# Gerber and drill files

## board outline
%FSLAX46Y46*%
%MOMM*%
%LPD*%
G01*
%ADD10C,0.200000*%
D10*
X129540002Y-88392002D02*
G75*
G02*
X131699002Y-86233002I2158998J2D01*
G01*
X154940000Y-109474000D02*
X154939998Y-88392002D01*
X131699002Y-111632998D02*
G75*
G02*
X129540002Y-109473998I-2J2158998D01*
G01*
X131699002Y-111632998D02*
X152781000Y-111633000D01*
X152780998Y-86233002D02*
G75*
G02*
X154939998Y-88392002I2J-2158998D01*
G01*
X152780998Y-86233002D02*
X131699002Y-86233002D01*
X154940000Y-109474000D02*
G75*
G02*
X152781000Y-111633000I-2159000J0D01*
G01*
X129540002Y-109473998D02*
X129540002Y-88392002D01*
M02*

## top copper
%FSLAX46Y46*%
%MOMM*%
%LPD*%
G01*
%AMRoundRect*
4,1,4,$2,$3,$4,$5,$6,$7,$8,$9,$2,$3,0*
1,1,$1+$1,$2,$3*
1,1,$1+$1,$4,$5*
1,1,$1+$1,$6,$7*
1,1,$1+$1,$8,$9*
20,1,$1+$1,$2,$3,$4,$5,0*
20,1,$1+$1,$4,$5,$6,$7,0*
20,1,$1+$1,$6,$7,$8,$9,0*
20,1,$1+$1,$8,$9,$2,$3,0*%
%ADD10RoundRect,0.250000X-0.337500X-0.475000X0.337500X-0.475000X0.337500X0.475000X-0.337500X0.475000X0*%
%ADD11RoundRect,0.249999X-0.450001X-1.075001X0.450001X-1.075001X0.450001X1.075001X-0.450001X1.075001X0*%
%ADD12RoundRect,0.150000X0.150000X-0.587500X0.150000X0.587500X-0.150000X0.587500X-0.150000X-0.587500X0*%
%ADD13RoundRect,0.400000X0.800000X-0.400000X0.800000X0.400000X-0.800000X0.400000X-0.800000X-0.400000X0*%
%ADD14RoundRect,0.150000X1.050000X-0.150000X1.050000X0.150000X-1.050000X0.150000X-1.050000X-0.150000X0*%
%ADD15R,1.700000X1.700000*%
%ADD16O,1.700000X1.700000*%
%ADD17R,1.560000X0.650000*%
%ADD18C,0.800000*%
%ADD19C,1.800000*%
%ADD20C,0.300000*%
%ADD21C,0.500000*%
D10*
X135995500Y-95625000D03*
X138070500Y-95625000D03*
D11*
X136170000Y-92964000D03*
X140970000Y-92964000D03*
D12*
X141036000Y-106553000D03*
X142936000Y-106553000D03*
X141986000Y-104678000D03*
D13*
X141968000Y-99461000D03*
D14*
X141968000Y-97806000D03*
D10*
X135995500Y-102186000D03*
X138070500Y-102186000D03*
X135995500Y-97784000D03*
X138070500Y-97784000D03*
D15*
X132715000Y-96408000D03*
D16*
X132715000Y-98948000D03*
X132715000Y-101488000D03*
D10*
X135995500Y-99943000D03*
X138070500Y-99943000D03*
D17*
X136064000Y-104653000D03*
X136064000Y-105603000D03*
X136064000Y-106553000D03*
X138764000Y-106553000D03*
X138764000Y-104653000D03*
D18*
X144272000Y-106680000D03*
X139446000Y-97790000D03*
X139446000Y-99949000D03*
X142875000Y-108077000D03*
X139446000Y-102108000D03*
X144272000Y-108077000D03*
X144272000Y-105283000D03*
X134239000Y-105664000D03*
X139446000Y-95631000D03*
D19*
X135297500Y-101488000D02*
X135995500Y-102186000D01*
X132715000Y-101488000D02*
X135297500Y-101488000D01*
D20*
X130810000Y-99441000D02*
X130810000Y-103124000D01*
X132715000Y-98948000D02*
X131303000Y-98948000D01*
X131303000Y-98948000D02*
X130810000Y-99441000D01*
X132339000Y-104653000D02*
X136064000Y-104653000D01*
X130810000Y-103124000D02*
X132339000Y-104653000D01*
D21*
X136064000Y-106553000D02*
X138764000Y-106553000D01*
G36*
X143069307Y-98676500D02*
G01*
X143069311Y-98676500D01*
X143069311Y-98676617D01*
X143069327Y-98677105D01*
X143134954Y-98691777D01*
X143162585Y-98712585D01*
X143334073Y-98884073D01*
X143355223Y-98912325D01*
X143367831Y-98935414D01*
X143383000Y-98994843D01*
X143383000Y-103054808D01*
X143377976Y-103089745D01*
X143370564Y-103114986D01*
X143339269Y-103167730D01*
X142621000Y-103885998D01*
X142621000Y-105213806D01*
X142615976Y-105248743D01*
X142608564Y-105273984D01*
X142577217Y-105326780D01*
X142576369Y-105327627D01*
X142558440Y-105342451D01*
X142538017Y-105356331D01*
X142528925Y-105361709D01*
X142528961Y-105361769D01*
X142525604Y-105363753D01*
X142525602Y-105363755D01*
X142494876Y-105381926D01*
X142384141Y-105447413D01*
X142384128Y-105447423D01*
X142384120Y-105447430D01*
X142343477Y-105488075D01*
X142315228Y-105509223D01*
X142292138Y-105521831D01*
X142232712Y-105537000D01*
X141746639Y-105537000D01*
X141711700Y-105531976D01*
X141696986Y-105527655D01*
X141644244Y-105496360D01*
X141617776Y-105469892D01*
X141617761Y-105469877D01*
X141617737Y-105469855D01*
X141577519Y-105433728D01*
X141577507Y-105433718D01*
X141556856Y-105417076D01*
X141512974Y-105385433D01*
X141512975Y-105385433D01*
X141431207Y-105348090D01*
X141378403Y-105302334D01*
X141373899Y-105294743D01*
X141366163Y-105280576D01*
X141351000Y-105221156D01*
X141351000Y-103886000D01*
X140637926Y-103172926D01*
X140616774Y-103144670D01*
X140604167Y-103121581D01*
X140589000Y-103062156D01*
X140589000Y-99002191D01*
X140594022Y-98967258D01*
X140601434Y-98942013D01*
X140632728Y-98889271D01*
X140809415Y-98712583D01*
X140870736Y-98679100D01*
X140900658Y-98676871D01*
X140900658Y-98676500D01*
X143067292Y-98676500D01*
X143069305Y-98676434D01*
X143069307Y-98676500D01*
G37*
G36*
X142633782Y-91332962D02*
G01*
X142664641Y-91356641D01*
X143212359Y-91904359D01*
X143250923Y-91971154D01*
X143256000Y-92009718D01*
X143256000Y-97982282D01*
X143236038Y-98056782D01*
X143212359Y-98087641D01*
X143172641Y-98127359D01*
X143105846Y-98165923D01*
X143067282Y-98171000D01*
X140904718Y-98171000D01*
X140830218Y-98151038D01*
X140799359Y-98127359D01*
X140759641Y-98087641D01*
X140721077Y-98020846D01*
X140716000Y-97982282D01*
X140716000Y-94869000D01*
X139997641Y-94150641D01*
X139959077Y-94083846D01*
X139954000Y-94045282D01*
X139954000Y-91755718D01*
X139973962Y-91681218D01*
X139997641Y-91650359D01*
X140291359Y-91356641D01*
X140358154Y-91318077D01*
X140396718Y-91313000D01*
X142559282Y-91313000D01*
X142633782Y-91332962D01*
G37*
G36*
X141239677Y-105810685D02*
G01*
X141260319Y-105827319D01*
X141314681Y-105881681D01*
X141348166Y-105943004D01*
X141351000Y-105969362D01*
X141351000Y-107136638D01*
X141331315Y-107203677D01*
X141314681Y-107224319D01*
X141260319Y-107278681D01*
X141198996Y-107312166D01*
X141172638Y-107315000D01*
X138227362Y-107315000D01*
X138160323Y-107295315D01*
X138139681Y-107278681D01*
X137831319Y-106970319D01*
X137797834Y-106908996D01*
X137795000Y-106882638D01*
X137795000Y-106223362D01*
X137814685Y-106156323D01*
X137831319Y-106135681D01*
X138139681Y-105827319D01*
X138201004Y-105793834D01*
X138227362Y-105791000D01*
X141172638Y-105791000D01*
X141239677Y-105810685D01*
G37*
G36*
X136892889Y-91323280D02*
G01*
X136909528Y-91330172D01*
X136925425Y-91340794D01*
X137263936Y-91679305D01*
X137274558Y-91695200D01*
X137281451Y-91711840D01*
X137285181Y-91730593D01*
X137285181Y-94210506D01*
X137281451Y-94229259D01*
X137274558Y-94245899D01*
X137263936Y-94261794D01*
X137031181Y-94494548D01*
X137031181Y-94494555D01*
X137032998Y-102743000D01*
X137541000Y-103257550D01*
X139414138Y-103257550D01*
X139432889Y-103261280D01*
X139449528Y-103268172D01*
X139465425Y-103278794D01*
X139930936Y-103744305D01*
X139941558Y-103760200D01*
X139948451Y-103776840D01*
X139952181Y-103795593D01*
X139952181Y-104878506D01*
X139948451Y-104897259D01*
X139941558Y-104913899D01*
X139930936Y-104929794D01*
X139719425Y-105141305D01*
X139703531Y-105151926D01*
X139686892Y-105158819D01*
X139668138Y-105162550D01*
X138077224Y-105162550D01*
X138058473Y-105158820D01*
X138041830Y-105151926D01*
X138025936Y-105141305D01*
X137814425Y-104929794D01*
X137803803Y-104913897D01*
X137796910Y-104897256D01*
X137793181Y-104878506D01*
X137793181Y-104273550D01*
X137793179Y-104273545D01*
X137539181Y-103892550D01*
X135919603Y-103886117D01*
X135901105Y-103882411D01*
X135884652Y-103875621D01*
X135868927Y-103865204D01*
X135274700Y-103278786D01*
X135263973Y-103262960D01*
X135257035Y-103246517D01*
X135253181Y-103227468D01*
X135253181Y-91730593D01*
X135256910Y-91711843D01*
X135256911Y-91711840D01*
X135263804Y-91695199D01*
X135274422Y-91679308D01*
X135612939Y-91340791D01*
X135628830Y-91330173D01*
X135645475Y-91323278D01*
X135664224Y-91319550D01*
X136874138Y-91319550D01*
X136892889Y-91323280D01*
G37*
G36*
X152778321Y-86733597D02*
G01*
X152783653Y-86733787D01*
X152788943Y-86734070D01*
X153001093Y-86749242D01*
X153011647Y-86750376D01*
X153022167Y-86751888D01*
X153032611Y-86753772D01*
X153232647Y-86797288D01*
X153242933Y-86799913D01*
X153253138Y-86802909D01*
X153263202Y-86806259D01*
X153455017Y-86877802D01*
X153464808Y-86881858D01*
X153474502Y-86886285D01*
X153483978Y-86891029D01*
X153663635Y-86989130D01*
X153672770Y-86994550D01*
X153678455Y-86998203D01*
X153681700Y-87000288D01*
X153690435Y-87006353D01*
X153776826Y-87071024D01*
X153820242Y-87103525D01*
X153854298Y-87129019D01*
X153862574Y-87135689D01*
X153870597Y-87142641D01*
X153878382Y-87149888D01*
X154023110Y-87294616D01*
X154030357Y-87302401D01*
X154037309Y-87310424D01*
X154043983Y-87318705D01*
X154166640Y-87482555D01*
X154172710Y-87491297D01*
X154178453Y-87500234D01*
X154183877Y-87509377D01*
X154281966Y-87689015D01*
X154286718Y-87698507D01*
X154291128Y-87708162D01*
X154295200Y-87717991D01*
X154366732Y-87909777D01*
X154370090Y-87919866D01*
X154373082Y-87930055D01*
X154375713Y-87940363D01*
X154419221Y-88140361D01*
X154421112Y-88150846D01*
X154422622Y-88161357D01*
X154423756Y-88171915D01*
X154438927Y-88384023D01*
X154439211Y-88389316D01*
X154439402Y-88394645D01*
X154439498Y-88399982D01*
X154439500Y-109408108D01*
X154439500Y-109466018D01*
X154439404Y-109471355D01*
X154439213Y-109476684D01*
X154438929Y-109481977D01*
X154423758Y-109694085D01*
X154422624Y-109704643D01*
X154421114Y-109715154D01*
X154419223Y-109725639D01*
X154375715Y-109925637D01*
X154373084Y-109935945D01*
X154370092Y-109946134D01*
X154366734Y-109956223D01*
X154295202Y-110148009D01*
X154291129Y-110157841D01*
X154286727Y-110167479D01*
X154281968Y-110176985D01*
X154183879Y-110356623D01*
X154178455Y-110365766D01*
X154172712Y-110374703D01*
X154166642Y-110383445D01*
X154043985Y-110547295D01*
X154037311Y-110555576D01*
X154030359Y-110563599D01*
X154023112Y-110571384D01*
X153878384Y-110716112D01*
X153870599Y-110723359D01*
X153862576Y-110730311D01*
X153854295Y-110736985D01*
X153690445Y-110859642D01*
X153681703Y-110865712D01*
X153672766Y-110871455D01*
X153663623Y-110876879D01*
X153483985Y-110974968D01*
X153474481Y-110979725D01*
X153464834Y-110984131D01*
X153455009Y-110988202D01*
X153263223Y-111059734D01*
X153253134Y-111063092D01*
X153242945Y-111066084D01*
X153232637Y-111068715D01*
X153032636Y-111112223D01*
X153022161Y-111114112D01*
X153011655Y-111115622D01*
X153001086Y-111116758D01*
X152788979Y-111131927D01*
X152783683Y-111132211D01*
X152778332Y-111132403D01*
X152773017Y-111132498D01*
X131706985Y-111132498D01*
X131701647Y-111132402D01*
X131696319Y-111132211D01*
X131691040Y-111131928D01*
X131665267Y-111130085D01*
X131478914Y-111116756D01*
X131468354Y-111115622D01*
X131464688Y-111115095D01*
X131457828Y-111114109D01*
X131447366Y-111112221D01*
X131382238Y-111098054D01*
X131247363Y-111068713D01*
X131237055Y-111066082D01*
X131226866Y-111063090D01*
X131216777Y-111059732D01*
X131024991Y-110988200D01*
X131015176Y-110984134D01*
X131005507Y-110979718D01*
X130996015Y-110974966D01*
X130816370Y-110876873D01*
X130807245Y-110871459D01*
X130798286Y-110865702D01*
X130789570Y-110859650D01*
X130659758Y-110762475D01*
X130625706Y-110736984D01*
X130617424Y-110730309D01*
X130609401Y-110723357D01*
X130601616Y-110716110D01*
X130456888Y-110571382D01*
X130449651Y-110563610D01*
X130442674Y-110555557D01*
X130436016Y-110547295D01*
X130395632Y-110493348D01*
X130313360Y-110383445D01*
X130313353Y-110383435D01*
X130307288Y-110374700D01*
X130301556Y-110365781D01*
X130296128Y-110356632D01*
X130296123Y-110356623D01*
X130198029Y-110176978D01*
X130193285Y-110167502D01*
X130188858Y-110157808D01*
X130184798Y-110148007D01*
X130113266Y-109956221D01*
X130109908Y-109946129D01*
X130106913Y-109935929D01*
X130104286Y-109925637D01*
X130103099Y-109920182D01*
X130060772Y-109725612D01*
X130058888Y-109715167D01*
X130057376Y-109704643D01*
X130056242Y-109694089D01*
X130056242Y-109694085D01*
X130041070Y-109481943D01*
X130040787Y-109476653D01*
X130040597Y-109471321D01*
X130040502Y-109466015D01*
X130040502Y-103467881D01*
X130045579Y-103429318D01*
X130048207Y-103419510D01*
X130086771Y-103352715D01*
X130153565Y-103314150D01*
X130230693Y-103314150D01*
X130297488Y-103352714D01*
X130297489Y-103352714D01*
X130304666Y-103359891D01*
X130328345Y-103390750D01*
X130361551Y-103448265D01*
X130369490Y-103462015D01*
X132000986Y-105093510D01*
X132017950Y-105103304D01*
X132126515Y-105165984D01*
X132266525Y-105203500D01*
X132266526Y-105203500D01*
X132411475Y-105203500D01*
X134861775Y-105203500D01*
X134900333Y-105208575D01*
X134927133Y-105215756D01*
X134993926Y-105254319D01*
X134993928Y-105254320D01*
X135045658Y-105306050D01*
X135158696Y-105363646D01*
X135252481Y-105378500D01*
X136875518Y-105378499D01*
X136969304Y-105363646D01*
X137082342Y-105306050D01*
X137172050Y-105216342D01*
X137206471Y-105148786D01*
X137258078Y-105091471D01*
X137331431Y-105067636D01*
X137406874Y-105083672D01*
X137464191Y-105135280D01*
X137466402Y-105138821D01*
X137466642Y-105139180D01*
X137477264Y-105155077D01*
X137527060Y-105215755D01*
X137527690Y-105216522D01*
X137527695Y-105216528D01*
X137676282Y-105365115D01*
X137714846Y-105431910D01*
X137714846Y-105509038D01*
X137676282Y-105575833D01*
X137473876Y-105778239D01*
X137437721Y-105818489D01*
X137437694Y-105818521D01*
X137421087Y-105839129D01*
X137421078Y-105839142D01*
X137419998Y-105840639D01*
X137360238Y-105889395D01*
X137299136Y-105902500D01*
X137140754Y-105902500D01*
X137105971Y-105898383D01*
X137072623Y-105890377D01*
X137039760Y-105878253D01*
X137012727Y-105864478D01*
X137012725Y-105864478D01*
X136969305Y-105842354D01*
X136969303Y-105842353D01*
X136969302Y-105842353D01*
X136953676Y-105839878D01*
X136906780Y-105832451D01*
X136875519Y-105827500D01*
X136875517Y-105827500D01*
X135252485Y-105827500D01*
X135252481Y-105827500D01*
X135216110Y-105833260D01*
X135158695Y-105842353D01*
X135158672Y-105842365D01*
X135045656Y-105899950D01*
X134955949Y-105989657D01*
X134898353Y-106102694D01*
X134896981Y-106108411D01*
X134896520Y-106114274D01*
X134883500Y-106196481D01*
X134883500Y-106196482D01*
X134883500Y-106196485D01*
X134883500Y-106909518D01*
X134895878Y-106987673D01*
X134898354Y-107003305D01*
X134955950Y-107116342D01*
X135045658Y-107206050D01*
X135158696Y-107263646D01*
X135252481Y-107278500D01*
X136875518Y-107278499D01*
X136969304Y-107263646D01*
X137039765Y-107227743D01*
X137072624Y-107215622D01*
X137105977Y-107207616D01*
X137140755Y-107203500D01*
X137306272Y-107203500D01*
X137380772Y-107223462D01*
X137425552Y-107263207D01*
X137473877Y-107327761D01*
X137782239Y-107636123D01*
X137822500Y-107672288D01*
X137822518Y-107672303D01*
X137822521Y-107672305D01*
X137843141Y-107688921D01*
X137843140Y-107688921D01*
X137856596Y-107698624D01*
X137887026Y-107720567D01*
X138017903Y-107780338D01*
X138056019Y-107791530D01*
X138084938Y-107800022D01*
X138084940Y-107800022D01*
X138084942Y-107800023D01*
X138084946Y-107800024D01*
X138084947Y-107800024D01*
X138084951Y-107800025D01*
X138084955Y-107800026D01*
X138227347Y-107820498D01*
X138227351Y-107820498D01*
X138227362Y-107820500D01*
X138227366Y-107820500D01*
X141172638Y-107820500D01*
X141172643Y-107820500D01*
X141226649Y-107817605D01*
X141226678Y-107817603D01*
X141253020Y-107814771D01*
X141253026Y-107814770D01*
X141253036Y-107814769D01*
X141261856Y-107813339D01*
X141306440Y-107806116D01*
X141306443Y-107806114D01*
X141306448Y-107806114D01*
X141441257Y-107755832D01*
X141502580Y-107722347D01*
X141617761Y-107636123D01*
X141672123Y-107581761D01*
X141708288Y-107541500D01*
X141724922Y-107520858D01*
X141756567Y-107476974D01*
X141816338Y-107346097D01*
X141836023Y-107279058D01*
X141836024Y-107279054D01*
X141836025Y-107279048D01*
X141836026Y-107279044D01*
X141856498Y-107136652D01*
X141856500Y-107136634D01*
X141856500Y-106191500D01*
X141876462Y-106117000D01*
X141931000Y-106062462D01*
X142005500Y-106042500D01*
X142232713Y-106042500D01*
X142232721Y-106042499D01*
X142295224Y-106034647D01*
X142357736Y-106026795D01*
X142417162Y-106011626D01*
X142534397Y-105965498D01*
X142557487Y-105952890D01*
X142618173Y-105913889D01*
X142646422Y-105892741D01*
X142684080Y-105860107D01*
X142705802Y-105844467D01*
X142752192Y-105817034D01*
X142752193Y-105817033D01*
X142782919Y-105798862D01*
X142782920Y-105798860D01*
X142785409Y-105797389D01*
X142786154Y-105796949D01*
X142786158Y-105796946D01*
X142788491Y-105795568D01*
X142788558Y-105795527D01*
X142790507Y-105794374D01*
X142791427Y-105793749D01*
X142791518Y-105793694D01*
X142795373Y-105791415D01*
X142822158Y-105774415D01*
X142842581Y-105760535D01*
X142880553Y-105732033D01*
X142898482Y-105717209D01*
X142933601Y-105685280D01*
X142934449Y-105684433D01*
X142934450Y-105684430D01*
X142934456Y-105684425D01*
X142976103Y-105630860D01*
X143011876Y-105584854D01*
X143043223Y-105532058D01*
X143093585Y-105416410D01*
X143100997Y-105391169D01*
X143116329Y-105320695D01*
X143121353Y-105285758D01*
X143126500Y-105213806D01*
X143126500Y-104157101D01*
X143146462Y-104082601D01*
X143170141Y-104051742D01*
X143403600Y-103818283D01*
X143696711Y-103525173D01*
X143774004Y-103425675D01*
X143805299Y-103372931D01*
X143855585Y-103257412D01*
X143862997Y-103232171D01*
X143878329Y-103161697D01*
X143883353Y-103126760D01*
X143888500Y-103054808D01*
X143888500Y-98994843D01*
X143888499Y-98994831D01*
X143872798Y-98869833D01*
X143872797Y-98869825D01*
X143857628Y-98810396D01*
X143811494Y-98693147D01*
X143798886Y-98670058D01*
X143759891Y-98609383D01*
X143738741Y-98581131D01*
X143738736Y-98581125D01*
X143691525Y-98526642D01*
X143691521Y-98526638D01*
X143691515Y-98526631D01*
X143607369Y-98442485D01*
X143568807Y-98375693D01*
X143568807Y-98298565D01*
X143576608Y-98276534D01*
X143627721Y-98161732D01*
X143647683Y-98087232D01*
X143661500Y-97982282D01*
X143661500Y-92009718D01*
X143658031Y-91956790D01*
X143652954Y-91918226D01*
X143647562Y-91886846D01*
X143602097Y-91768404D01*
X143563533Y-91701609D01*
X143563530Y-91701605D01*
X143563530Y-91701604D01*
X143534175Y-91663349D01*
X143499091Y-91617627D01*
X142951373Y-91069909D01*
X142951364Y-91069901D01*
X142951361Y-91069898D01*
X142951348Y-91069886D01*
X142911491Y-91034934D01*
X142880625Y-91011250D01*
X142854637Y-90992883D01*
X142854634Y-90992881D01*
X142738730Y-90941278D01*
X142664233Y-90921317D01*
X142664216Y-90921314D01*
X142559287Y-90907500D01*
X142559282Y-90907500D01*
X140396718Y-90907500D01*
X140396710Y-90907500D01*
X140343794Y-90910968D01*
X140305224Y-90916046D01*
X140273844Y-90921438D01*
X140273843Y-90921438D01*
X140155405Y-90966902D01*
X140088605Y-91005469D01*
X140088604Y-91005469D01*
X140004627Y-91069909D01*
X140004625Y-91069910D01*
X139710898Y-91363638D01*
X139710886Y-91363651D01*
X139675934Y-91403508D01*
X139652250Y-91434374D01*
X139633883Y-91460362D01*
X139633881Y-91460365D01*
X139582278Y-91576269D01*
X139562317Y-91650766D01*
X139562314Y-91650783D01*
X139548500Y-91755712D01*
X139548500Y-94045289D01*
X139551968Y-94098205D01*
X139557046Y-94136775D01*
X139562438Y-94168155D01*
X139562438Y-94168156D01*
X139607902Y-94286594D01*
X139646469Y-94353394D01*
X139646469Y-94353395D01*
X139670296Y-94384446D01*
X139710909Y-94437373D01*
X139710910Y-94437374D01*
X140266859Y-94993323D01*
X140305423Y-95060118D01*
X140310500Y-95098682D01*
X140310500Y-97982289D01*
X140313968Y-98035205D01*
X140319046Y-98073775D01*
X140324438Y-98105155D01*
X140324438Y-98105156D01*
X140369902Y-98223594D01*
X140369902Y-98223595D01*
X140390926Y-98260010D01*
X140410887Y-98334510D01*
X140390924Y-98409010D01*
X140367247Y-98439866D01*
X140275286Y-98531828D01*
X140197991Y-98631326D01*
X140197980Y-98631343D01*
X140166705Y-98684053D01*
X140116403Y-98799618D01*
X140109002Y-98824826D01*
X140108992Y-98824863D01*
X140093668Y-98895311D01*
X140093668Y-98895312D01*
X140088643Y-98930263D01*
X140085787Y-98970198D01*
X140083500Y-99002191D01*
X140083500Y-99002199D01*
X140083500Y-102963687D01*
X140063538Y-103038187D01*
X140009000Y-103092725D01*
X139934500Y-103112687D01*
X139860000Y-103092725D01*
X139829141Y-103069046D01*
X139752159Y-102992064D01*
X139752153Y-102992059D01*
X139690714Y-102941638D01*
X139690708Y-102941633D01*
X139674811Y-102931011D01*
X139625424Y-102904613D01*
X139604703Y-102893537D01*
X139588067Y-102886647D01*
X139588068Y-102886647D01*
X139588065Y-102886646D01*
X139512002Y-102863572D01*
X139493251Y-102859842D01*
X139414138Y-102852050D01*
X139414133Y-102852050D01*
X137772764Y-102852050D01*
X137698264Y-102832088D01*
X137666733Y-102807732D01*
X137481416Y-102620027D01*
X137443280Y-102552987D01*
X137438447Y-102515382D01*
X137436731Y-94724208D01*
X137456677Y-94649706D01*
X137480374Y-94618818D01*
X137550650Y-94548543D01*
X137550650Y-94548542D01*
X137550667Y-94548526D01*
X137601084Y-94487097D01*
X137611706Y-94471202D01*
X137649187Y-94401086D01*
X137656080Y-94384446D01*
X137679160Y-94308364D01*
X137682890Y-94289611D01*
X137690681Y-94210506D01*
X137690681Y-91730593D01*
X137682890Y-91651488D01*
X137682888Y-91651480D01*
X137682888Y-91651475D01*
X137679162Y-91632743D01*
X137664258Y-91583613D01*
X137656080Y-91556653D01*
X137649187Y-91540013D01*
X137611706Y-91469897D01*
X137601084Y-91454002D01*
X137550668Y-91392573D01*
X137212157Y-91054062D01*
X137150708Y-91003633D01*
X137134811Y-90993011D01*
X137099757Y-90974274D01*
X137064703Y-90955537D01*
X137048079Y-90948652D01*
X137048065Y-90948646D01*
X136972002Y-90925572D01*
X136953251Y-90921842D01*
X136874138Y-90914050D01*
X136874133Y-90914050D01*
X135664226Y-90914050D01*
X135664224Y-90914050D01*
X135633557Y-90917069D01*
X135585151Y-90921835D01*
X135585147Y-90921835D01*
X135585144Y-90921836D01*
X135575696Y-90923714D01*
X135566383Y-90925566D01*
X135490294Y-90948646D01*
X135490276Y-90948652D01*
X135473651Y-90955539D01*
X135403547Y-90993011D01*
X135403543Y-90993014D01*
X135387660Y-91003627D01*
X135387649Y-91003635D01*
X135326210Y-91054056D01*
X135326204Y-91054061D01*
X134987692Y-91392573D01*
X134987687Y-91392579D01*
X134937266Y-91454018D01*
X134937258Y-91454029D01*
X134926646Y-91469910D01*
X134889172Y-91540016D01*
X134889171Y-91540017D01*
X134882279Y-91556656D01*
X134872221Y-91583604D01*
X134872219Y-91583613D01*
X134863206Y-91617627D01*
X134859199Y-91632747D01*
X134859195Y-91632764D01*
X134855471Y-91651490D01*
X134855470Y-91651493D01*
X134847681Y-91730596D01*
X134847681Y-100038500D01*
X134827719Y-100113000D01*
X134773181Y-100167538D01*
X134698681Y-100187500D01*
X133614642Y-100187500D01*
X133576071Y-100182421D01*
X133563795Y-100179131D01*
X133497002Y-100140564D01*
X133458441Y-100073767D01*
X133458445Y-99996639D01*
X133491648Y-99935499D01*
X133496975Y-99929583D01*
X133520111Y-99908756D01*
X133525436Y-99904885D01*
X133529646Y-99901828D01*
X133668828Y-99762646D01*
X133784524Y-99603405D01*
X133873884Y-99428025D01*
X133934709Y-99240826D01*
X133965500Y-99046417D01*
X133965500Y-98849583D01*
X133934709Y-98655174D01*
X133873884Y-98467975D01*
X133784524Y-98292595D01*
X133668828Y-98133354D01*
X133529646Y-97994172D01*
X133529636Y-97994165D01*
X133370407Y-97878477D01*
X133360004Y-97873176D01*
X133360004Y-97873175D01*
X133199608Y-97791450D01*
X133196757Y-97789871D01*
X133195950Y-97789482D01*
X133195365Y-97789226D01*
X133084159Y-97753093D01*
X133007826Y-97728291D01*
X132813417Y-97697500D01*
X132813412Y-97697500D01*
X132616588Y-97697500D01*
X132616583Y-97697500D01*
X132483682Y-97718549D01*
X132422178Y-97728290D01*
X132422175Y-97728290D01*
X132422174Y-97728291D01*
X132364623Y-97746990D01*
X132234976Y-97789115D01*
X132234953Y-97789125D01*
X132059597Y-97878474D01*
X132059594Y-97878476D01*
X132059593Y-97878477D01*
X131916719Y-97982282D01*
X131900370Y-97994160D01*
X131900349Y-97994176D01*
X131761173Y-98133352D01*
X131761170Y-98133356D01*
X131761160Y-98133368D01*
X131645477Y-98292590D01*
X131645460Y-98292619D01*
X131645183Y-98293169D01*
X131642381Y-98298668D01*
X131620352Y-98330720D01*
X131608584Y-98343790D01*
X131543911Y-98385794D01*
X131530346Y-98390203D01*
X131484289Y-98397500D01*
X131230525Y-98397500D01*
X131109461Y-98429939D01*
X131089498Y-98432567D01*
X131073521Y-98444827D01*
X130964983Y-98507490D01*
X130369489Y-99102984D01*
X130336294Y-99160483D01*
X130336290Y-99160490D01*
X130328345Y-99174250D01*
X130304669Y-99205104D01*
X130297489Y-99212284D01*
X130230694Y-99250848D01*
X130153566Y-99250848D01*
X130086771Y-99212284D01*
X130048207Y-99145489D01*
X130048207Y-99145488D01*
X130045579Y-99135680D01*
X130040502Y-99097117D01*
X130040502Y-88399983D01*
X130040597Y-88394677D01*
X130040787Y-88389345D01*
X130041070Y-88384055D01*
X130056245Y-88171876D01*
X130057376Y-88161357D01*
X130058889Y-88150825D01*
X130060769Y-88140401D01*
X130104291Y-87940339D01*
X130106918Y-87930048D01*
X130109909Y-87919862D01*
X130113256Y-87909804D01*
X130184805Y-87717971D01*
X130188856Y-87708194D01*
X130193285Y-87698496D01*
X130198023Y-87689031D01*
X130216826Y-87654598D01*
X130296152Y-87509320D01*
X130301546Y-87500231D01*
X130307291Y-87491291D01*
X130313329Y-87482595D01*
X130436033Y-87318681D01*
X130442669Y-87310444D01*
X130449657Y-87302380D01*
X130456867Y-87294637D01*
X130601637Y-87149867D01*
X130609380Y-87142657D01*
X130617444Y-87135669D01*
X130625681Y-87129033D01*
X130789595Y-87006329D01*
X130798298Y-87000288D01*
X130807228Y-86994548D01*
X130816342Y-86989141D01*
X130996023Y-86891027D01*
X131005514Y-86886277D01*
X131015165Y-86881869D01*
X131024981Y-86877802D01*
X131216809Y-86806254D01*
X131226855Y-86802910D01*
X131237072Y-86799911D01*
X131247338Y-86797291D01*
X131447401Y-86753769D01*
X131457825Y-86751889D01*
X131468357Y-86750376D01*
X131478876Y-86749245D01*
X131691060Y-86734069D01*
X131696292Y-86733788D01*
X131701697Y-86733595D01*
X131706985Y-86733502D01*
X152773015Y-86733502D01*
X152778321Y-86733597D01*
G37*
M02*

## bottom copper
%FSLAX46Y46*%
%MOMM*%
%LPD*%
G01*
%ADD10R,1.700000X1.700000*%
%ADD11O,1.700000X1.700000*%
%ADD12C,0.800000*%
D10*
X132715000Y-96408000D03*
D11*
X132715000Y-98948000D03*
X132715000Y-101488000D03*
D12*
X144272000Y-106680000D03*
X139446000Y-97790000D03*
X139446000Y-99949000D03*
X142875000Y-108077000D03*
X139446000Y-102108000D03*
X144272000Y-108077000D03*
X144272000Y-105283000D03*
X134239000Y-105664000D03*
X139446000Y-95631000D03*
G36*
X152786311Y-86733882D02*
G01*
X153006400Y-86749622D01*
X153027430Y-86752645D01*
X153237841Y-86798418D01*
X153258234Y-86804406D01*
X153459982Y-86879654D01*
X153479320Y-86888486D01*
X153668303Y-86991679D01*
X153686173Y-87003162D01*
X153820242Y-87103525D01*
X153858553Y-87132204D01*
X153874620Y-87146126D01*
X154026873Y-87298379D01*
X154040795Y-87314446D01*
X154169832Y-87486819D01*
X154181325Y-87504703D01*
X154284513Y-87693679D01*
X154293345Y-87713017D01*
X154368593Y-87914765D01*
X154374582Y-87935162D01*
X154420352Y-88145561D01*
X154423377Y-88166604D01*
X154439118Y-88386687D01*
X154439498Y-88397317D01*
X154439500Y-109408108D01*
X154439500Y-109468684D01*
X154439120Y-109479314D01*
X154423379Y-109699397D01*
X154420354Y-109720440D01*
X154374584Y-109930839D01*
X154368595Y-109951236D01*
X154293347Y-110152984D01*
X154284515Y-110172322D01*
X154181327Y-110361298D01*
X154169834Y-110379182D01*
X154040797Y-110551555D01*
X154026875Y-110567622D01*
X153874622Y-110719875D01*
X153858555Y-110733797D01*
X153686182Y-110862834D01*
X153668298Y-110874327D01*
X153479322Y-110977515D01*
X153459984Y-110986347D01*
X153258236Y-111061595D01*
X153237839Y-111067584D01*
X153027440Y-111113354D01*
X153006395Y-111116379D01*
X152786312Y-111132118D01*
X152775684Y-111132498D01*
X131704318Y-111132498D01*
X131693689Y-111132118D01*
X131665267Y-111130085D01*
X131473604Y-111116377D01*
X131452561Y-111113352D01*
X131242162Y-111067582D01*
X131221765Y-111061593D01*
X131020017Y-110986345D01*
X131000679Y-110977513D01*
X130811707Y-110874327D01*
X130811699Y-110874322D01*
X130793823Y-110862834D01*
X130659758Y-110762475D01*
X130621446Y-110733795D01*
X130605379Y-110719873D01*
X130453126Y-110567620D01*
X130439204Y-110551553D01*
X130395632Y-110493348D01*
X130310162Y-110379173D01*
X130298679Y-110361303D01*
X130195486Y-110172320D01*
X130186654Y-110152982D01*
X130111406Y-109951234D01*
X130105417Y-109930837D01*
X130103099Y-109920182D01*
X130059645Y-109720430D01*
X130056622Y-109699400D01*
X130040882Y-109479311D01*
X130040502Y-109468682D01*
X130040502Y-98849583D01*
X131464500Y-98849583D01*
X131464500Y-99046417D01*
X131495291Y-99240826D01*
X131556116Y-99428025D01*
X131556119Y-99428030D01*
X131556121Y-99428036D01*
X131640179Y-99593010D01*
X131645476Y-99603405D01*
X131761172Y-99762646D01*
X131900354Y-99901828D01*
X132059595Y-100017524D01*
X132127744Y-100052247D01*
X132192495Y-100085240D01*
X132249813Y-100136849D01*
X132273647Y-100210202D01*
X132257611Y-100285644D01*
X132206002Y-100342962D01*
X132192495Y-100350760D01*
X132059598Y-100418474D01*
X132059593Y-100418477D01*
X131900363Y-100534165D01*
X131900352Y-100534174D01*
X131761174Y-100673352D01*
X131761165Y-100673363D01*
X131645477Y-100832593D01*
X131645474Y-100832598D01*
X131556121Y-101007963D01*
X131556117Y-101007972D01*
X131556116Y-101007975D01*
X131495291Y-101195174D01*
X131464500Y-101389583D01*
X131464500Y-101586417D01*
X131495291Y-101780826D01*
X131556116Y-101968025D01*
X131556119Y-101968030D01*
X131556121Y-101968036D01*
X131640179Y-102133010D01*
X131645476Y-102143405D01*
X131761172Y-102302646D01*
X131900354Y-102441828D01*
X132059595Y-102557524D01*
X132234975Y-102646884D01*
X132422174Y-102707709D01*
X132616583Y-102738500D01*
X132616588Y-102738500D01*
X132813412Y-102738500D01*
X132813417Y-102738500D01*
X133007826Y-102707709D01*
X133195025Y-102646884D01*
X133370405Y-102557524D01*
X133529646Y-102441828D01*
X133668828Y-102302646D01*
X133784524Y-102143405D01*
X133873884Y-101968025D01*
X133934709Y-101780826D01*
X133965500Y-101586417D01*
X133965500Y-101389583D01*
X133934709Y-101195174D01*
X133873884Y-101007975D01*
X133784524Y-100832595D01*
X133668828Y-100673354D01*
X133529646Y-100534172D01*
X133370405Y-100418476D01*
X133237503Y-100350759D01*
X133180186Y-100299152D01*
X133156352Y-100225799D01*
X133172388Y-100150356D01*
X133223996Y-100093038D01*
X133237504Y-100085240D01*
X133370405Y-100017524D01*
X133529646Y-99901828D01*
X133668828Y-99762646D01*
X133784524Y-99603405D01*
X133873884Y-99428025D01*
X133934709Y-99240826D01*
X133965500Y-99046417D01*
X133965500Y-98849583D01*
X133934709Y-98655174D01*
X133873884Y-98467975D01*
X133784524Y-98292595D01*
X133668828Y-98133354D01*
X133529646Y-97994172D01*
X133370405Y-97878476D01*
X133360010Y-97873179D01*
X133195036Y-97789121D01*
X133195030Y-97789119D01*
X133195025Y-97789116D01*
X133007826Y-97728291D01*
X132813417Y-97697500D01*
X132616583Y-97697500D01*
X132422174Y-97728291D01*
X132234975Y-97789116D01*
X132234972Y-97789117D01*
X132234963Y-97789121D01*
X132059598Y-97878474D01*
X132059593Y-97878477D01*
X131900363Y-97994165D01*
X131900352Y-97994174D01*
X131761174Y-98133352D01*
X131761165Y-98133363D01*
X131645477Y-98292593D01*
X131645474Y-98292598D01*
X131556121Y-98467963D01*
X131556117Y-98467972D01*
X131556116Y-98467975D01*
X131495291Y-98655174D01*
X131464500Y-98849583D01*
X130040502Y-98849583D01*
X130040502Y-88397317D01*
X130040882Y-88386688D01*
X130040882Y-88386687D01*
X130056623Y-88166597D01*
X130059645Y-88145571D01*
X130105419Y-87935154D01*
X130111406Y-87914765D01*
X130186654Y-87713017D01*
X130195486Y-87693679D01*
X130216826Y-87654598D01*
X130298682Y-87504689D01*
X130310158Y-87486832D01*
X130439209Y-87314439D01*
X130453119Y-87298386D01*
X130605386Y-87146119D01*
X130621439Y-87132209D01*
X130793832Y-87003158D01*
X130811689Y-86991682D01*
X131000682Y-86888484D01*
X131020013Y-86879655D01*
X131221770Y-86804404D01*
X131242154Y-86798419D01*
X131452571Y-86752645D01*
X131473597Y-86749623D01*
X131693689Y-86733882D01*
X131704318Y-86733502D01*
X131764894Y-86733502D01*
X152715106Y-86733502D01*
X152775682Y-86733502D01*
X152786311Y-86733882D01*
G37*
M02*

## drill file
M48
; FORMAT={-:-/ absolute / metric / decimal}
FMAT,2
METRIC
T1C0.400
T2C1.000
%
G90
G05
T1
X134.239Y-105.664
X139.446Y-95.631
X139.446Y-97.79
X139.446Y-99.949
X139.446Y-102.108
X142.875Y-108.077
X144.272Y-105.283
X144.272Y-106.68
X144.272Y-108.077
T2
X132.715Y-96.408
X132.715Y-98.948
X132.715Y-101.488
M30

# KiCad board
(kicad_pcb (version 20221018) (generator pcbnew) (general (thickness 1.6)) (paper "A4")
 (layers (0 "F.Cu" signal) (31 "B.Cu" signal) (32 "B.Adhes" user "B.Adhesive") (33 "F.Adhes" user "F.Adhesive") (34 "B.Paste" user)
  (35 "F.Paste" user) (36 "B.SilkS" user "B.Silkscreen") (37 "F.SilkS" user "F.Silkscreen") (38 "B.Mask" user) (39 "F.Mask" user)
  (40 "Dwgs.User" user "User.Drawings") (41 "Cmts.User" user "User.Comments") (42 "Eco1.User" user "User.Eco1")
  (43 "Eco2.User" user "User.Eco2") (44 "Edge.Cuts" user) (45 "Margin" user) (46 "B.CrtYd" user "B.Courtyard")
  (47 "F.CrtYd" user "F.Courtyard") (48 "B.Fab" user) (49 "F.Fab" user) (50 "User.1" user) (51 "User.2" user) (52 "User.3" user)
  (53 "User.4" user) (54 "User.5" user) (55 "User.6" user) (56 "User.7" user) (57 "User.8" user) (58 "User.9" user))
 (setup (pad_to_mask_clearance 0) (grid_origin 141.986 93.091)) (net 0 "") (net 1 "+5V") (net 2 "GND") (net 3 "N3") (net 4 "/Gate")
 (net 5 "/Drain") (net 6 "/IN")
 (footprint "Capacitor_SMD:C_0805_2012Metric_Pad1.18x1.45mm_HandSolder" (layer "F.Cu") (at 137.033 95.625)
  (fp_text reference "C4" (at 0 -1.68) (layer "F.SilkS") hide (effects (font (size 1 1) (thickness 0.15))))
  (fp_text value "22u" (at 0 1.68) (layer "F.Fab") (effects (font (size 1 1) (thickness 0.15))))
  (pad "1" smd roundrect (at -1.0375 0) (size 1.175 1.45) (layers "F.Cu" "F.Paste" "F.Mask") (roundrect_rratio 0.2127659574) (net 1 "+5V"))
  (pad "2" smd roundrect (at 1.0375 0) (size 1.175 1.45) (layers "F.Cu" "F.Paste" "F.Mask") (roundrect_rratio 0.2127659574) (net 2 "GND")))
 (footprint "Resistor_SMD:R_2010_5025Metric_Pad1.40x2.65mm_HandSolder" (layer "F.Cu") (at 138.57 92.964)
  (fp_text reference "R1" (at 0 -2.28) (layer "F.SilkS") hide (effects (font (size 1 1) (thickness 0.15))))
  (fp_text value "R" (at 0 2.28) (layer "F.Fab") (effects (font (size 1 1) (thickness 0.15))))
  (pad "1" smd roundrect (at -2.4 0) (size 1.4 2.65) (layers "F.Cu" "F.Paste" "F.Mask") (roundrect_rratio 0.1785707143) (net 1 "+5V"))
  (pad "2" smd roundrect (at 2.4 0) (size 1.4 2.65) (layers "F.Cu" "F.Paste" "F.Mask") (roundrect_rratio 0.1785707143) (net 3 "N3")))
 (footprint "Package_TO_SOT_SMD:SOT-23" (layer "F.Cu") (at 141.986 105.6155 90)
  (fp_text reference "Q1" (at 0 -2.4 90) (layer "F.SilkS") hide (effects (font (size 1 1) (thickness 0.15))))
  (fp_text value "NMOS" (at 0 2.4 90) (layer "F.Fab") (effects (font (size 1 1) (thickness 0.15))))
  (pad "1" smd roundrect (at -0.9375 -0.95 90) (size 1.475 0.6) (layers "F.Cu" "F.Paste" "F.Mask") (roundrect_rratio 0.25) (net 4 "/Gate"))
  (pad "2" smd roundrect (at -0.9375 0.95 90) (size 1.475 0.6) (layers "F.Cu" "F.Paste" "F.Mask") (roundrect_rratio 0.25) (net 2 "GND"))
  (pad "3" smd roundrect (at 0.9375 0 90) (size 1.475 0.6) (layers "F.Cu" "F.Paste" "F.Mask") (roundrect_rratio 0.25) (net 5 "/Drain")))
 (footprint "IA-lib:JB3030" (layer "F.Cu") (at 141.968 98.661 90)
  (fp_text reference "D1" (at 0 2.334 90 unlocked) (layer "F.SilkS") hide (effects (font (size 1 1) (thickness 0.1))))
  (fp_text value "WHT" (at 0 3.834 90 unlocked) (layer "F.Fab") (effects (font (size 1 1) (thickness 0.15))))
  (pad "1" smd roundrect (at -0.8 0 90) (size 1.6 2.4) (layers "F.Cu" "F.Paste" "F.Mask") (roundrect_rratio 0.25) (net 5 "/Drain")
   (thermal_bridge_angle 45))
  (pad "2" smd roundrect (at 0.855 0 90) (size 0.6 2.4) (layers "F.Cu" "F.Paste" "F.Mask") (roundrect_rratio 0.25) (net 3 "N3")
   (thermal_bridge_angle 45)))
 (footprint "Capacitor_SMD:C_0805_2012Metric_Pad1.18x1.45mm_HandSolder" (layer "F.Cu") (at 137.033 102.186)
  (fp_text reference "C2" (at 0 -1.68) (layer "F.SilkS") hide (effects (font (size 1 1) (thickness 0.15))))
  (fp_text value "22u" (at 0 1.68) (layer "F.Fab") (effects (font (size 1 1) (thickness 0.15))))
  (pad "1" smd roundrect (at -1.0375 0) (size 1.175 1.45) (layers "F.Cu" "F.Paste" "F.Mask") (roundrect_rratio 0.2127659574) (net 1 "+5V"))
  (pad "2" smd roundrect (at 1.0375 0) (size 1.175 1.45) (layers "F.Cu" "F.Paste" "F.Mask") (roundrect_rratio 0.2127659574) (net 2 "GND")))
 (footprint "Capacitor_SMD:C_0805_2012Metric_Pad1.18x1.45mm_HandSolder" (layer "F.Cu") (at 137.033 97.784)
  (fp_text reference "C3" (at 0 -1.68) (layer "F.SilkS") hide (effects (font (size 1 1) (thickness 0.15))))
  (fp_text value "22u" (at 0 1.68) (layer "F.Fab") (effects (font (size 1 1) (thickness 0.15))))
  (pad "1" smd roundrect (at -1.0375 0) (size 1.175 1.45) (layers "F.Cu" "F.Paste" "F.Mask") (roundrect_rratio 0.2127659574) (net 1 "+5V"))
  (pad "2" smd roundrect (at 1.0375 0) (size 1.175 1.45) (layers "F.Cu" "F.Paste" "F.Mask") (roundrect_rratio 0.2127659574) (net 2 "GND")))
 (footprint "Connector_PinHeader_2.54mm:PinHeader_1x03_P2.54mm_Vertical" (layer "F.Cu") (at 132.715 96.408)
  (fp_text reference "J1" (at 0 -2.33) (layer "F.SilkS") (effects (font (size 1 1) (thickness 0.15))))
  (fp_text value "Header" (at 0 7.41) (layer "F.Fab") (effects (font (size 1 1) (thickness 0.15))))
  (pad "1" thru_hole rect (at 0 0) (size 1.7 1.7) (drill 1) (layers "*.Cu" "*.Mask") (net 2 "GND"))
  (pad "2" thru_hole oval (at 0 2.54) (size 1.7 1.7) (drill 1) (layers "*.Cu" "*.Mask") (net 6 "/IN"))
  (pad "3" thru_hole oval (at 0 5.08) (size 1.7 1.7) (drill 1) (layers "*.Cu" "*.Mask") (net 1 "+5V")))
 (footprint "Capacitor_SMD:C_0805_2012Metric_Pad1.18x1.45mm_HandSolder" (layer "F.Cu") (at 137.033 99.943)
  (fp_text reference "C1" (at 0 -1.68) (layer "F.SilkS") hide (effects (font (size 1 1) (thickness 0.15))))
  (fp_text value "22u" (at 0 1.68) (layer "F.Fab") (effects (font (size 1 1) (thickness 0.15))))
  (pad "1" smd roundrect (at -1.0375 0) (size 1.175 1.45) (layers "F.Cu" "F.Paste" "F.Mask") (roundrect_rratio 0.2127659574) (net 1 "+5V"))
  (pad "2" smd roundrect (at 1.0375 0) (size 1.175 1.45) (layers "F.Cu" "F.Paste" "F.Mask") (roundrect_rratio 0.2127659574) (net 2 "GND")))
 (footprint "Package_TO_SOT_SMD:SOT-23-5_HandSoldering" (layer "F.Cu") (at 137.414 105.603)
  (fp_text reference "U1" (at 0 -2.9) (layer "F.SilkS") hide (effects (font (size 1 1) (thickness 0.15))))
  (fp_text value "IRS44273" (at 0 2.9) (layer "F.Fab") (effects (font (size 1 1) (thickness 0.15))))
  (pad "1" smd rect (at -1.35 -0.95) (size 1.56 0.65) (layers "F.Cu" "F.Paste" "F.Mask") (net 6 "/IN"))
  (pad "2" smd rect (at -1.35 0) (size 1.56 0.65) (layers "F.Cu" "F.Paste" "F.Mask") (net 2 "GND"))
  (pad "3" smd rect (at -1.35 0.95) (size 1.56 0.65) (layers "F.Cu" "F.Paste" "F.Mask") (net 4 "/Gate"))
  (pad "4" smd rect (at 1.35 0.95) (size 1.56 0.65) (layers "F.Cu" "F.Paste" "F.Mask") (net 4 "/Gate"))
  (pad "5" smd rect (at 1.35 -0.95) (size 1.56 0.65) (layers "F.Cu" "F.Paste" "F.Mask") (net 1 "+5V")))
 (gr_arc (start 129.540002 88.392002) (mid 130.172358 86.865358) (end 131.699002 86.233002) (stroke (width 0.2) (type default))
  (layer "Edge.Cuts"))
 (gr_line (start 154.94 109.474) (end 154.939998 88.392002) (stroke (width 0.2) (type default)) (layer "Edge.Cuts"))
 (gr_arc (start 131.699002 111.632998) (mid 130.172358 111.000642) (end 129.540002 109.473998) (stroke (width 0.2) (type default))
  (layer "Edge.Cuts"))
 (gr_line (start 131.699002 111.632998) (end 152.781 111.633) (stroke (width 0.2) (type default)) (layer "Edge.Cuts"))
 (gr_arc (start 152.780998 86.233002) (mid 154.307642 86.865358) (end 154.939998 88.392002) (stroke (width 0.2) (type default))
  (layer "Edge.Cuts"))
 (gr_line (start 152.780998 86.233002) (end 131.699002 86.233002) (stroke (width 0.2) (type default)) (layer "Edge.Cuts"))
 (gr_arc (start 154.94 109.474) (mid 154.307644 111.000644) (end 152.781 111.633) (stroke (width 0.2) (type default)) (layer "Edge.Cuts"))
 (gr_line (start 129.540002 109.473998) (end 129.540002 88.392002) (stroke (width 0.2) (type default)) (layer "Edge.Cuts"))
 (segment (start 135.2975 101.488) (end 135.9955 102.186) (width 1.8) (layer "F.Cu") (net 1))
 (segment (start 132.715 101.488) (end 135.2975 101.488) (width 1.8) (layer "F.Cu") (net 1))
 (via (at 144.272 106.68) (size 0.8) (drill 0.4) (layers "F.Cu" "B.Cu") (free) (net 2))
 (via (at 139.446 97.79) (size 0.8) (drill 0.4) (layers "F.Cu" "B.Cu") (free) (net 2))
 (via (at 139.446 99.949) (size 0.8) (drill 0.4) (layers "F.Cu" "B.Cu") (free) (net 2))
 (via (at 142.875 108.077) (size 0.8) (drill 0.4) (layers "F.Cu" "B.Cu") (free) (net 2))
 (via (at 139.446 102.108) (size 0.8) (drill 0.4) (layers "F.Cu" "B.Cu") (free) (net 2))
 (via (at 144.272 108.077) (size 0.8) (drill 0.4) (layers "F.Cu" "B.Cu") (free) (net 2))
 (via (at 144.272 105.283) (size 0.8) (drill 0.4) (layers "F.Cu" "B.Cu") (free) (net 2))
 (via (at 134.239 105.664) (size 0.8) (drill 0.4) (layers "F.Cu" "B.Cu") (free) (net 2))
 (via (at 139.446 95.631) (size 0.8) (drill 0.4) (layers "F.Cu" "B.Cu") (free) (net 2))
 (segment (start 130.81 99.441) (end 130.81 103.124) (width 0.3) (layer "F.Cu") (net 6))
 (segment (start 132.715 98.948) (end 131.303 98.948) (width 0.3) (layer "F.Cu") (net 6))
 (segment (start 131.303 98.948) (end 130.81 99.441) (width 0.3) (layer "F.Cu") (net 6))
 (segment (start 132.339 104.653) (end 136.064 104.653) (width 0.3) (layer "F.Cu") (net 6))
 (segment (start 130.81 103.124) (end 132.339 104.653) (width 0.3) (layer "F.Cu") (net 6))
 (segment (start 136.064 106.553) (end 138.764 106.553) (width 0.5) (layer "F.Cu") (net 4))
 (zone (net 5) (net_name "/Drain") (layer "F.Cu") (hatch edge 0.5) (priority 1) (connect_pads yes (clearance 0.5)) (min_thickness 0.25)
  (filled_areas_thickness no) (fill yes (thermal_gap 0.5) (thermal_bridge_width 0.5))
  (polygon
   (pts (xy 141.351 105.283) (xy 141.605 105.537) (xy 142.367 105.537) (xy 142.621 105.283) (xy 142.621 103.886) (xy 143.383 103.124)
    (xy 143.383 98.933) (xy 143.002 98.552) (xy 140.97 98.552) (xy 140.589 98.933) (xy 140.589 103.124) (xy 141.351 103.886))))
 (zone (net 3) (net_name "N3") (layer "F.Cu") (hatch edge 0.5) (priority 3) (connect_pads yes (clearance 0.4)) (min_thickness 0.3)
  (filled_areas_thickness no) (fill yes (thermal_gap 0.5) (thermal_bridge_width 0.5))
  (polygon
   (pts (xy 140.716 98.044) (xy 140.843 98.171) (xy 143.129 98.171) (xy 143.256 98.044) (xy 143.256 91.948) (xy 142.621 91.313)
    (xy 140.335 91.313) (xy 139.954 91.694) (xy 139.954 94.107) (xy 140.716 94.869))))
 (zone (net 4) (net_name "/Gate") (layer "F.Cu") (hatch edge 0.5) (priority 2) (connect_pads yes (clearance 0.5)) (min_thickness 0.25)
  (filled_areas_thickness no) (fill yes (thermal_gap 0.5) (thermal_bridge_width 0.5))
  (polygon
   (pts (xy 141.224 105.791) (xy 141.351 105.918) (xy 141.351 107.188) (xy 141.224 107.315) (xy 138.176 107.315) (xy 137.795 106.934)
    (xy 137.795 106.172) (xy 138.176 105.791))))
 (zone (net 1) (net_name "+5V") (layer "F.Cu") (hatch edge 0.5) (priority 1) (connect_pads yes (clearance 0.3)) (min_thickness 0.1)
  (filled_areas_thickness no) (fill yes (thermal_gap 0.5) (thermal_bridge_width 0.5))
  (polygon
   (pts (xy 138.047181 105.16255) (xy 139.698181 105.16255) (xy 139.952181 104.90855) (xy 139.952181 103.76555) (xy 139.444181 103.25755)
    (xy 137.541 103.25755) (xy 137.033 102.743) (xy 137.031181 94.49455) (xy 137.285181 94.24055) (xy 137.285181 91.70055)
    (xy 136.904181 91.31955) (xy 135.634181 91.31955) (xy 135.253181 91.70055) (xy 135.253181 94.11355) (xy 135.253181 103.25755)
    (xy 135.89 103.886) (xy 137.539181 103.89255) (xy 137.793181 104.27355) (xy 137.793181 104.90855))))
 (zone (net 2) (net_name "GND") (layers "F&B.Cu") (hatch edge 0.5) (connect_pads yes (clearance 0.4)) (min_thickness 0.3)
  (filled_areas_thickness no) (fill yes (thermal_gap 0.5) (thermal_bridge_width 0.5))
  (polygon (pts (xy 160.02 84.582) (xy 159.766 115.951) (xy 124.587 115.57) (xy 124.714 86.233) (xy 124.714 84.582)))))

